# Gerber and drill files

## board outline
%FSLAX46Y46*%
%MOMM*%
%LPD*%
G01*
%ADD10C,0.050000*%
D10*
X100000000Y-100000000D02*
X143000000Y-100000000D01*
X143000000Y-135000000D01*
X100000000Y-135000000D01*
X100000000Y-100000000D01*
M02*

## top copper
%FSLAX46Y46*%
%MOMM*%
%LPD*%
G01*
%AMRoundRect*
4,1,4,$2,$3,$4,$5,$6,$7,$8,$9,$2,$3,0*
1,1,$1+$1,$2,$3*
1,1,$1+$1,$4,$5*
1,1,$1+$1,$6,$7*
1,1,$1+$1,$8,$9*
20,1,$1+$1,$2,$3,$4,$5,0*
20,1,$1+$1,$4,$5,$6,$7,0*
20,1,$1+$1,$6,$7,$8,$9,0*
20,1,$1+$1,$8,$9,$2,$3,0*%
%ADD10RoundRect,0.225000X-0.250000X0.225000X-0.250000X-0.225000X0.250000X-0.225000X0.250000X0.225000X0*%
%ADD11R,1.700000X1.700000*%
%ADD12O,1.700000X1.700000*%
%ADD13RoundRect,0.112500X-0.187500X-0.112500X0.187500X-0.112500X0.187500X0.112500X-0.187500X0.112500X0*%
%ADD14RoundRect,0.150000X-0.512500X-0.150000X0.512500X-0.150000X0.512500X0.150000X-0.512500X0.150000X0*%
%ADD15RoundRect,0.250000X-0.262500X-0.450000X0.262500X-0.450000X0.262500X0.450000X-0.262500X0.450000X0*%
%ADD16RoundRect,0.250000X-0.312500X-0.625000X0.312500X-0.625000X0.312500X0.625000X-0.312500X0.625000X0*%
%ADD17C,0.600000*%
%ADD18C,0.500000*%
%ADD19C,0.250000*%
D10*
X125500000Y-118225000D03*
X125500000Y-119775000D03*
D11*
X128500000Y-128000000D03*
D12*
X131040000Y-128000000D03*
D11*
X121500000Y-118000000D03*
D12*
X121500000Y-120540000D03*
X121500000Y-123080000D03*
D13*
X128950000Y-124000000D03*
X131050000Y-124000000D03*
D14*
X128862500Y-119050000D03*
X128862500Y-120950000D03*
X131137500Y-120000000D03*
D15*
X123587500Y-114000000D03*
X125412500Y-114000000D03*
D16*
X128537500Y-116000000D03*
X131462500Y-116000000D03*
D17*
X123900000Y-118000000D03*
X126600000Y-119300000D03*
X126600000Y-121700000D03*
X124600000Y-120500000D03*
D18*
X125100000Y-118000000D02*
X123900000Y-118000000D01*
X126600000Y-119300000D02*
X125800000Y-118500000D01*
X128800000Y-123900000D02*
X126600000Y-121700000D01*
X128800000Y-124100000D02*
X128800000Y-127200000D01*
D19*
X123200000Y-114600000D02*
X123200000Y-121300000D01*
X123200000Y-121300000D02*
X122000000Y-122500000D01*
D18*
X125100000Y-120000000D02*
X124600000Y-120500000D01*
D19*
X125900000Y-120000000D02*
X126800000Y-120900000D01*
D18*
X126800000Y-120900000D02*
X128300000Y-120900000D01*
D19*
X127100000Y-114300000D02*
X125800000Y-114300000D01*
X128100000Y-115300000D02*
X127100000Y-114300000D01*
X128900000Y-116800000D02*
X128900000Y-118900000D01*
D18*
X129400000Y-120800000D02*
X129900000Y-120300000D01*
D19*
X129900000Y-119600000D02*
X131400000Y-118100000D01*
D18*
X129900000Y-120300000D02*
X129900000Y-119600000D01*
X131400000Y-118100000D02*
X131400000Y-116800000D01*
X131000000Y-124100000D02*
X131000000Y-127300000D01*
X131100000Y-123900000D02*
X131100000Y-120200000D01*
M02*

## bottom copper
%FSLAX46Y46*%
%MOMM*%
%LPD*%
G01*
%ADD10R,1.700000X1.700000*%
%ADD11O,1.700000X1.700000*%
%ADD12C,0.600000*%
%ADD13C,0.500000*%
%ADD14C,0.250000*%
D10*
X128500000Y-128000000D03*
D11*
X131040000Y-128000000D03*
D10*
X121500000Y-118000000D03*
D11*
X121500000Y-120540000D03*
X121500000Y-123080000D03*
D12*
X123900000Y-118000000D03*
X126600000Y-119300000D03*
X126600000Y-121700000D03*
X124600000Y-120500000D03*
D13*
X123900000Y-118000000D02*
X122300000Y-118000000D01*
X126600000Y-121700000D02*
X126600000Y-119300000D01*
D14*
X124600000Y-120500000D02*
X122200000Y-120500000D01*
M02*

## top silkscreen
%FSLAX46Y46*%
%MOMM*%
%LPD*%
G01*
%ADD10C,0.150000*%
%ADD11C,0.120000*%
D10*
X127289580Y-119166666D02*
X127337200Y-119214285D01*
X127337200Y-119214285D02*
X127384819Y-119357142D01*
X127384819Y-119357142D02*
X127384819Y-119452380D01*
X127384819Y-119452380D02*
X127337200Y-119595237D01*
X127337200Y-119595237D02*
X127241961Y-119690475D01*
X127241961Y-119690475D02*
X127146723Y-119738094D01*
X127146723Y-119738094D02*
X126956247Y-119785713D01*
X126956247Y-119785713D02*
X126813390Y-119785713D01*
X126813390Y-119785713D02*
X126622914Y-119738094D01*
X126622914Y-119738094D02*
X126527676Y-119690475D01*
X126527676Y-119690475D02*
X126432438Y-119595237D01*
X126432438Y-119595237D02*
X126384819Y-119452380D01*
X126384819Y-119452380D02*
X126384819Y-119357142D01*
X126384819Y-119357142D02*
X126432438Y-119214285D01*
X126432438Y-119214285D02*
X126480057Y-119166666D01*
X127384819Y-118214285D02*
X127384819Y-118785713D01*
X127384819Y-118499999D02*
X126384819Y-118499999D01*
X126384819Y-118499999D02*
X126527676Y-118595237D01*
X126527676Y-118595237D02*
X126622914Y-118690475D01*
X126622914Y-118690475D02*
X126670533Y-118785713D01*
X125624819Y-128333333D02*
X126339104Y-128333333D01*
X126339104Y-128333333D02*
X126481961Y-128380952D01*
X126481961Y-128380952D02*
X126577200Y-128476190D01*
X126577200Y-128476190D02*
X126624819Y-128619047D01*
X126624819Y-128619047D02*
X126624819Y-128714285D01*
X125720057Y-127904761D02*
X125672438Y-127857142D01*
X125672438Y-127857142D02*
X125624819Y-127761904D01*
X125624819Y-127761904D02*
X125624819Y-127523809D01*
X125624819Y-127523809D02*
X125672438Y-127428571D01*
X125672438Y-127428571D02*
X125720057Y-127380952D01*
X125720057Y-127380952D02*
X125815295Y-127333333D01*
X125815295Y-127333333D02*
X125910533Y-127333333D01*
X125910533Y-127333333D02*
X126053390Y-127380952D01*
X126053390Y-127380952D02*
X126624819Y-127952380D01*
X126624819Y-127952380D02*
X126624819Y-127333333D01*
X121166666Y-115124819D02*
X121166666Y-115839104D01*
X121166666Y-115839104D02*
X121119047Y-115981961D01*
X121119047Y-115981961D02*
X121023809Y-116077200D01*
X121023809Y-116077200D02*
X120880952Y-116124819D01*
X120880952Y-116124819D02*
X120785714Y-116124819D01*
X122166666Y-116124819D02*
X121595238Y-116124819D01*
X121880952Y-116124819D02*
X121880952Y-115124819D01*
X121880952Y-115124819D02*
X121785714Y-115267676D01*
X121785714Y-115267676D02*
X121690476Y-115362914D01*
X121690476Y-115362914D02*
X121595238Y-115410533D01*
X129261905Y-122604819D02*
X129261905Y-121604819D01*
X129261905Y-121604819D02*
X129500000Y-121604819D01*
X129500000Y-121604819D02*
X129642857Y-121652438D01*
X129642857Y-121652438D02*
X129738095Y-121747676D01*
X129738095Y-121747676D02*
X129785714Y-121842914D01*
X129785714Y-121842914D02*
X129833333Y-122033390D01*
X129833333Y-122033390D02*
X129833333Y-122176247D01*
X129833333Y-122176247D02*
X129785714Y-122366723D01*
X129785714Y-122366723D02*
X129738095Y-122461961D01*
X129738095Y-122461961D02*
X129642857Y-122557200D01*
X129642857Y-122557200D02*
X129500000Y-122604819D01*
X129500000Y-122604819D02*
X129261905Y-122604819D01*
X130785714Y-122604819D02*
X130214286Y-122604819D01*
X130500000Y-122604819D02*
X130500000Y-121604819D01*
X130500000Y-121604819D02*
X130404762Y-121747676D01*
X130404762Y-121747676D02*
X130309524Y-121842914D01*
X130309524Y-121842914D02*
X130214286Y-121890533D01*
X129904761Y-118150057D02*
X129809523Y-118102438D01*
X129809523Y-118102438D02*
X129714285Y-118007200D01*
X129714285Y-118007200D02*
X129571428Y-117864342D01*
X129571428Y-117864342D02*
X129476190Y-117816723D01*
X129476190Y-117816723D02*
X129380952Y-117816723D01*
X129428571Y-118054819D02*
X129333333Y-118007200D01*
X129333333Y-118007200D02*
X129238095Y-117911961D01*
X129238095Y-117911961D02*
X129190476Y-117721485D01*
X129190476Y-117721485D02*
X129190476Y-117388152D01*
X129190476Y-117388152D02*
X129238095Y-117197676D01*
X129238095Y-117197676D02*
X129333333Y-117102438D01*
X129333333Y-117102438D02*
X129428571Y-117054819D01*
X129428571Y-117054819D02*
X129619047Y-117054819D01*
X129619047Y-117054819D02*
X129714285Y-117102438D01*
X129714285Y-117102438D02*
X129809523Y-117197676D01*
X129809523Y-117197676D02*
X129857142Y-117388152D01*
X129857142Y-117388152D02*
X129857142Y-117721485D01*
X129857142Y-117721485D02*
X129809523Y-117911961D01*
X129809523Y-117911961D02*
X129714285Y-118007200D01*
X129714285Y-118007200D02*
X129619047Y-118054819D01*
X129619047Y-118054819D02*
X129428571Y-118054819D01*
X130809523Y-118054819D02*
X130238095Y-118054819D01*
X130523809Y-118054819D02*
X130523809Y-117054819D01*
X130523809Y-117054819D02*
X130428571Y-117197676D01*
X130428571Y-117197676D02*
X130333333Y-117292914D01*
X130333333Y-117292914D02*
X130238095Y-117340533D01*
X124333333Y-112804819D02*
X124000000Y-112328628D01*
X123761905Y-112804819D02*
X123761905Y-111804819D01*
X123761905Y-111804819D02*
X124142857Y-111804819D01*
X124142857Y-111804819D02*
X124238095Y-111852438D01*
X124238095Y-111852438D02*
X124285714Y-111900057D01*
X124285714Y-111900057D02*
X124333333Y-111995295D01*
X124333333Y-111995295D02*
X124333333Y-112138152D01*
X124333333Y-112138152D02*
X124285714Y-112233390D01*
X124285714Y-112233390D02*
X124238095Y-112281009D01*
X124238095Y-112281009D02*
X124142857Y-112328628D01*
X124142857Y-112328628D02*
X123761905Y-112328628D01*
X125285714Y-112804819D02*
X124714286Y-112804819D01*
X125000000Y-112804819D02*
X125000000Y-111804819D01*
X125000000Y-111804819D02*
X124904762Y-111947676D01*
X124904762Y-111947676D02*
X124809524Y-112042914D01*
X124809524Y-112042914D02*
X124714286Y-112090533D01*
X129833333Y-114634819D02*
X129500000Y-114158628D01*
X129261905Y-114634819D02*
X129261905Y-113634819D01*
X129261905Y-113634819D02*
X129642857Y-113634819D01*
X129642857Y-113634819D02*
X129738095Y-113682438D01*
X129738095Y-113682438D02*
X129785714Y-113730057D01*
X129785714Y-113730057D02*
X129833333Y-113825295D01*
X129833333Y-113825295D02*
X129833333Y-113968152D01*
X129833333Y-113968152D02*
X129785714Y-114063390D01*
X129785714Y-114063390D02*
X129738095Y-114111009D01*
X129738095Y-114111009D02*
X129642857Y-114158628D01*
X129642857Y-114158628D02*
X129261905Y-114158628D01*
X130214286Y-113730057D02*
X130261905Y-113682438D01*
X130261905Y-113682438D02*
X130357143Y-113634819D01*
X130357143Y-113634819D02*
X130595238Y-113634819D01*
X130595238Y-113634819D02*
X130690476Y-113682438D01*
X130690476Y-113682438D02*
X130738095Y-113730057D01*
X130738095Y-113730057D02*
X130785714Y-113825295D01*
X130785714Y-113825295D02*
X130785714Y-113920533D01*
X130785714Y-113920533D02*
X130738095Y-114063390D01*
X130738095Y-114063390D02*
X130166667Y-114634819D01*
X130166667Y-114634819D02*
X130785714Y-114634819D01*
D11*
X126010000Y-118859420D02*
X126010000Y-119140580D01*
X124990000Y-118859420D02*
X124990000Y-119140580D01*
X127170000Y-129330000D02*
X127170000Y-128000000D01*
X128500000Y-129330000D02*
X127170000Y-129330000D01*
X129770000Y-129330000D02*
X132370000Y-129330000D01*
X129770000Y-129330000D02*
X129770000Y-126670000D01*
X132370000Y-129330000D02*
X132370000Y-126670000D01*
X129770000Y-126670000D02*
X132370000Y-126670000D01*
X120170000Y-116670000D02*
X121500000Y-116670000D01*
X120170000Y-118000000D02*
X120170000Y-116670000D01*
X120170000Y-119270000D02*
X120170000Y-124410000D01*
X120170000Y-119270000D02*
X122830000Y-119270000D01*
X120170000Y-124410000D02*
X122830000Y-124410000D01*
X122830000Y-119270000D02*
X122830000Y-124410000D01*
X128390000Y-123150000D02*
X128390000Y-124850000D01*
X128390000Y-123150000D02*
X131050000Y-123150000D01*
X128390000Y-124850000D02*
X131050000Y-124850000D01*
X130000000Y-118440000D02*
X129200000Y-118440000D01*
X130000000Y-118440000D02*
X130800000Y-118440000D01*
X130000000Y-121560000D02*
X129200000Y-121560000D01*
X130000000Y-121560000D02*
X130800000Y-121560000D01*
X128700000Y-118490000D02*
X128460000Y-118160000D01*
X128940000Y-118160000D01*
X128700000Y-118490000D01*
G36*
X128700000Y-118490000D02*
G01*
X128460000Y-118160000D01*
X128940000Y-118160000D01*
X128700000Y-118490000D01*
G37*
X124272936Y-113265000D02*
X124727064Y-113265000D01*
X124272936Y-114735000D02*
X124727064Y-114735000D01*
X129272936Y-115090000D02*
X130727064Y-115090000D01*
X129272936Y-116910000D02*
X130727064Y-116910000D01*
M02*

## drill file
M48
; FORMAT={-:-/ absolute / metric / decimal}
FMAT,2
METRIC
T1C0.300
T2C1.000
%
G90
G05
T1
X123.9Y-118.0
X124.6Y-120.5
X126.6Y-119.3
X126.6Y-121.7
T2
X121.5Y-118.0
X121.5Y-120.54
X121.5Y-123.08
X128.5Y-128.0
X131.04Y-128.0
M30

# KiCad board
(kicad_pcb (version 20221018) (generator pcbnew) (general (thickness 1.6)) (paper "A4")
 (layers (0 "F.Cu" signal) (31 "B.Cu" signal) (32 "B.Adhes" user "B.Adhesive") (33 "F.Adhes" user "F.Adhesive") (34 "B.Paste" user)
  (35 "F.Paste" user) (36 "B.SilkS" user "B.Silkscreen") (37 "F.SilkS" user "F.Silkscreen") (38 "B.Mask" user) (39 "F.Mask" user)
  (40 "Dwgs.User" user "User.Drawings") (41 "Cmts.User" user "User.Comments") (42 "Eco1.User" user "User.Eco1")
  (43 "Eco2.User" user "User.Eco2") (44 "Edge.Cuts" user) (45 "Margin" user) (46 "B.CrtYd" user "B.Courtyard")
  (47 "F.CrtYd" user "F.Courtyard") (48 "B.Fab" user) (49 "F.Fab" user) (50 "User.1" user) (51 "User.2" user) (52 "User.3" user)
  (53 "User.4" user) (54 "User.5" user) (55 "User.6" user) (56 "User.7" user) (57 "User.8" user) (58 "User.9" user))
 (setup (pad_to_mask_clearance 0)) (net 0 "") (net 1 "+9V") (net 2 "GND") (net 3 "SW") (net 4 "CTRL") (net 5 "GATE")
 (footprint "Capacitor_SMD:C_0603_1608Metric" (layer "F.Cu") (at 125.5 119 -90)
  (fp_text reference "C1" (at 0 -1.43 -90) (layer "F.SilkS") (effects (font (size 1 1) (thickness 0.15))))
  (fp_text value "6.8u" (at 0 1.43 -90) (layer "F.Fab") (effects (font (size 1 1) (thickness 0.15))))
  (fp_line (start -0.14058 -0.51) (end 0.14058 -0.51) (stroke (width 0.12) (type solid)) (layer "F.SilkS"))
  (fp_line (start -0.14058 0.51) (end 0.14058 0.51) (stroke (width 0.12) (type solid)) (layer "F.SilkS"))
  (pad "1" smd roundrect (at -0.775 0 270) (size 0.9 0.95) (layers "F.Cu" "F.Paste" "F.Mask") (roundrect_rratio 0.25) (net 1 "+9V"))
  (pad "2" smd roundrect (at 0.775 0 270) (size 0.9 0.95) (layers "F.Cu" "F.Paste" "F.Mask") (roundrect_rratio 0.25) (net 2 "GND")))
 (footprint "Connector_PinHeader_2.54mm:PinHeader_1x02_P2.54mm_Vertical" (layer "F.Cu") (at 128.5 128 90)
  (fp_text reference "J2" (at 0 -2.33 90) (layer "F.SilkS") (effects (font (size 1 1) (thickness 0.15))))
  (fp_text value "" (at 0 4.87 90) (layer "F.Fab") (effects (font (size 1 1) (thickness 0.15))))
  (fp_line (start -1.33 -1.33) (end 0 -1.33) (stroke (width 0.12) (type solid)) (layer "F.SilkS"))
  (fp_line (start -1.33 0) (end -1.33 -1.33) (stroke (width 0.12) (type solid)) (layer "F.SilkS"))
  (fp_line (start -1.33 1.27) (end -1.33 3.87) (stroke (width 0.12) (type solid)) (layer "F.SilkS"))
  (fp_line (start -1.33 1.27) (end 1.33 1.27) (stroke (width 0.12) (type solid)) (layer "F.SilkS"))
  (fp_line (start -1.33 3.87) (end 1.33 3.87) (stroke (width 0.12) (type solid)) (layer "F.SilkS"))
  (fp_line (start 1.33 1.27) (end 1.33 3.87) (stroke (width 0.12) (type solid)) (layer "F.SilkS"))
  (pad "1" thru_hole rect (at 0 0 90) (size 1.7 1.7) (drill 1) (layers "*.Cu" "*.Mask") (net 1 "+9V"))
  (pad "2" thru_hole oval (at 0 2.54 90) (size 1.7 1.7) (drill 1) (layers "*.Cu" "*.Mask") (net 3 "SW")))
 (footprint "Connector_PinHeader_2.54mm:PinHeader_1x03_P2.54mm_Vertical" (layer "F.Cu") (at 121.5 118)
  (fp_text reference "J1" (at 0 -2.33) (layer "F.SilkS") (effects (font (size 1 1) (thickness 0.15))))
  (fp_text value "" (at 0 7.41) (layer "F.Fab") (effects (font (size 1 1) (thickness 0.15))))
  (fp_line (start -1.33 -1.33) (end 0 -1.33) (stroke (width 0.12) (type solid)) (layer "F.SilkS"))
  (fp_line (start -1.33 0) (end -1.33 -1.33) (stroke (width 0.12) (type solid)) (layer "F.SilkS"))
  (fp_line (start -1.33 1.27) (end -1.33 6.41) (stroke (width 0.12) (type solid)) (layer "F.SilkS"))
  (fp_line (start -1.33 1.27) (end 1.33 1.27) (stroke (width 0.12) (type solid)) (layer "F.SilkS"))
  (fp_line (start -1.33 6.41) (end 1.33 6.41) (stroke (width 0.12) (type solid)) (layer "F.SilkS"))
  (fp_line (start 1.33 1.27) (end 1.33 6.41) (stroke (width 0.12) (type solid)) (layer "F.SilkS"))
  (pad "1" thru_hole rect (at 0 0) (size 1.7 1.7) (drill 1) (layers "*.Cu" "*.Mask") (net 1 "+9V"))
  (pad "2" thru_hole oval (at 0 2.54) (size 1.7 1.7) (drill 1) (layers "*.Cu" "*.Mask") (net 2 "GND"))
  (pad "3" thru_hole oval (at 0 5.08) (size 1.7 1.7) (drill 1) (layers "*.Cu" "*.Mask") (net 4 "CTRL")))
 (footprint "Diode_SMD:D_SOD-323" (layer "F.Cu") (at 130 124)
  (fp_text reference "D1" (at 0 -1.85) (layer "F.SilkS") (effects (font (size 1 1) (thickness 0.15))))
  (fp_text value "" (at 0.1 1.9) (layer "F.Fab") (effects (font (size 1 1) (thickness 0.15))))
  (fp_line (start -1.61 -0.85) (end -1.61 0.85) (stroke (width 0.12) (type solid)) (layer "F.SilkS"))
  (fp_line (start -1.61 -0.85) (end 1.05 -0.85) (stroke (width 0.12) (type solid)) (layer "F.SilkS"))
  (fp_line (start -1.61 0.85) (end 1.05 0.85) (stroke (width 0.12) (type solid)) (layer "F.SilkS"))
  (pad "1" smd roundrect (at -1.05 0) (size 0.6 0.45) (layers "F.Cu" "F.Paste" "F.Mask") (roundrect_rratio 0.25) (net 1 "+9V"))
  (pad "2" smd roundrect (at 1.05 0) (size 0.6 0.45) (layers "F.Cu" "F.Paste" "F.Mask") (roundrect_rratio 0.25) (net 3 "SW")))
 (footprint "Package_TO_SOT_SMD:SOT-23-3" (layer "F.Cu") (at 130 120)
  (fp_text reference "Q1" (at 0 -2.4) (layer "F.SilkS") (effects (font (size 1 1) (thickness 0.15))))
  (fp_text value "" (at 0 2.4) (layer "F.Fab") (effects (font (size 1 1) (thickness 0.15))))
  (fp_line (start 0 -1.56) (end -0.8 -1.56) (stroke (width 0.12) (type solid)) (layer "F.SilkS"))
  (fp_line (start 0 -1.56) (end 0.8 -1.56) (stroke (width 0.12) (type solid)) (layer "F.SilkS"))
  (fp_line (start 0 1.56) (end -0.8 1.56) (stroke (width 0.12) (type solid)) (layer "F.SilkS"))
  (fp_line (start 0 1.56) (end 0.8 1.56) (stroke (width 0.12) (type solid)) (layer "F.SilkS"))
  (fp_poly
   (pts (xy -1.3 -1.51) (xy -1.54 -1.84) (xy -1.06 -1.84) (xy -1.3 -1.51)) (stroke (width 0.12) (type solid)) (fill solid) (layer "F.SilkS"))
  (pad "1" smd roundrect (at -1.1375 -0.95) (size 1.325 0.6) (layers "F.Cu" "F.Paste" "F.Mask") (roundrect_rratio 0.25) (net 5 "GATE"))
  (pad "2" smd roundrect (at -1.1375 0.95) (size 1.325 0.6) (layers "F.Cu" "F.Paste" "F.Mask") (roundrect_rratio 0.25) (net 2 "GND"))
  (pad "3" smd roundrect (at 1.1375 0) (size 1.325 0.6) (layers "F.Cu" "F.Paste" "F.Mask") (roundrect_rratio 0.25) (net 3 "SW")))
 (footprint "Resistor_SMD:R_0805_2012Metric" (layer "F.Cu") (at 124.5 114)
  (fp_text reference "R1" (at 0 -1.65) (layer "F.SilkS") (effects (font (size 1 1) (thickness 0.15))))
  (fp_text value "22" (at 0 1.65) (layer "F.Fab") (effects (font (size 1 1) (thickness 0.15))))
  (fp_line (start -0.227064 -0.735) (end 0.227064 -0.735) (stroke (width 0.12) (type solid)) (layer "F.SilkS"))
  (fp_line (start -0.227064 0.735) (end 0.227064 0.735) (stroke (width 0.12) (type solid)) (layer "F.SilkS"))
  (pad "1" smd roundrect (at -0.9125 0) (size 1.025 1.4) (layers "F.Cu" "F.Paste" "F.Mask") (roundrect_rratio 0.243902) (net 4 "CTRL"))
  (pad "2" smd roundrect (at 0.9125 0) (size 1.025 1.4) (layers "F.Cu" "F.Paste" "F.Mask") (roundrect_rratio 0.243902) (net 5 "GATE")))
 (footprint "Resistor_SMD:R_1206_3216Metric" (layer "F.Cu") (at 130 116)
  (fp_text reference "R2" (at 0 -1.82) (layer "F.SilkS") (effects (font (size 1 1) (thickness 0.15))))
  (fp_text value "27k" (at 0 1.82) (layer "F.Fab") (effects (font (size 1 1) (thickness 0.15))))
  (fp_line (start -0.727064 -0.91) (end 0.727064 -0.91) (stroke (width 0.12) (type solid)) (layer "F.SilkS"))
  (fp_line (start -0.727064 0.91) (end 0.727064 0.91) (stroke (width 0.12) (type solid)) (layer "F.SilkS"))
  (pad "1" smd roundrect (at -1.4625 0) (size 1.125 1.75) (layers "F.Cu" "F.Paste" "F.Mask") (roundrect_rratio 0.222222) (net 5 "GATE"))
  (pad "2" smd roundrect (at 1.4625 0) (size 1.125 1.75) (layers "F.Cu" "F.Paste" "F.Mask") (roundrect_rratio 0.222222) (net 2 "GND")))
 (gr_rect (start 100 100) (end 143 135) (stroke (width 0.05) (type default)) (fill none) (layer "Edge.Cuts"))
 (segment (start 125.1 118) (end 123.9 118) (width 0.5) (layer "F.Cu") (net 1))
 (segment (start 126.6 119.3) (end 125.8 118.5) (width 0.5) (layer "F.Cu") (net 1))
 (segment (start 128.8 123.9) (end 126.6 121.7) (width 0.5) (layer "F.Cu") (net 1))
 (segment (start 128.8 124.1) (end 128.8 127.2) (width 0.5) (layer "F.Cu") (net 1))
 (via (at 123.9 118) (size 0.6) (drill 0.3) (layers "F.Cu" "B.Cu") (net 1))
 (via (at 126.6 119.3) (size 0.6) (drill 0.3) (layers "F.Cu" "B.Cu") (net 1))
 (via (at 126.6 121.7) (size 0.6) (drill 0.3) (layers "F.Cu" "B.Cu") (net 1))
 (segment (start 123.2 114.6) (end 123.2 121.3) (width 0.25) (layer "F.Cu") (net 4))
 (segment (start 123.2 121.3) (end 122 122.5) (width 0.25) (layer "F.Cu") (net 4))
 (segment (start 123.9 118) (end 122.3 118) (width 0.5) (layer "B.Cu") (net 1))
 (segment (start 125.1 120) (end 124.6 120.5) (width 0.5) (layer "F.Cu") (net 2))
 (segment (start 125.9 120) (end 126.8 120.9) (width 0.25) (layer "F.Cu") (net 2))
 (segment (start 126.6 121.7) (end 126.6 119.3) (width 0.5) (layer "B.Cu") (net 1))
 (segment (start 126.8 120.9) (end 128.3 120.9) (width 0.5) (layer "F.Cu") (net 2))
 (segment (start 127.1 114.3) (end 125.8 114.3) (width 0.25) (layer "F.Cu") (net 5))
 (segment (start 128.1 115.3) (end 127.1 114.3) (width 0.25) (layer "F.Cu") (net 5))
 (segment (start 128.9 116.8) (end 128.9 118.9) (width 0.25) (layer "F.Cu") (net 5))
 (segment (start 129.4 120.8) (end 129.9 120.3) (width 0.5) (layer "F.Cu") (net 2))
 (segment (start 129.9 119.6) (end 131.4 118.1) (width 0.25) (layer "F.Cu") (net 2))
 (segment (start 129.9 120.3) (end 129.9 119.6) (width 0.5) (layer "F.Cu") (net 2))
 (segment (start 131.4 118.1) (end 131.4 116.8) (width 0.5) (layer "F.Cu") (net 2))
 (via (at 124.6 120.5) (size 0.6) (drill 0.3) (layers "F.Cu" "B.Cu") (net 2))
 (segment (start 124.6 120.5) (end 122.2 120.5) (width 0.25) (layer "B.Cu") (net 2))
 (segment (start 131 124.1) (end 131 127.3) (width 0.5) (layer "F.Cu") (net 3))
 (segment (start 131.1 123.9) (end 131.1 120.2) (width 0.5) (layer "F.Cu") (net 3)))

